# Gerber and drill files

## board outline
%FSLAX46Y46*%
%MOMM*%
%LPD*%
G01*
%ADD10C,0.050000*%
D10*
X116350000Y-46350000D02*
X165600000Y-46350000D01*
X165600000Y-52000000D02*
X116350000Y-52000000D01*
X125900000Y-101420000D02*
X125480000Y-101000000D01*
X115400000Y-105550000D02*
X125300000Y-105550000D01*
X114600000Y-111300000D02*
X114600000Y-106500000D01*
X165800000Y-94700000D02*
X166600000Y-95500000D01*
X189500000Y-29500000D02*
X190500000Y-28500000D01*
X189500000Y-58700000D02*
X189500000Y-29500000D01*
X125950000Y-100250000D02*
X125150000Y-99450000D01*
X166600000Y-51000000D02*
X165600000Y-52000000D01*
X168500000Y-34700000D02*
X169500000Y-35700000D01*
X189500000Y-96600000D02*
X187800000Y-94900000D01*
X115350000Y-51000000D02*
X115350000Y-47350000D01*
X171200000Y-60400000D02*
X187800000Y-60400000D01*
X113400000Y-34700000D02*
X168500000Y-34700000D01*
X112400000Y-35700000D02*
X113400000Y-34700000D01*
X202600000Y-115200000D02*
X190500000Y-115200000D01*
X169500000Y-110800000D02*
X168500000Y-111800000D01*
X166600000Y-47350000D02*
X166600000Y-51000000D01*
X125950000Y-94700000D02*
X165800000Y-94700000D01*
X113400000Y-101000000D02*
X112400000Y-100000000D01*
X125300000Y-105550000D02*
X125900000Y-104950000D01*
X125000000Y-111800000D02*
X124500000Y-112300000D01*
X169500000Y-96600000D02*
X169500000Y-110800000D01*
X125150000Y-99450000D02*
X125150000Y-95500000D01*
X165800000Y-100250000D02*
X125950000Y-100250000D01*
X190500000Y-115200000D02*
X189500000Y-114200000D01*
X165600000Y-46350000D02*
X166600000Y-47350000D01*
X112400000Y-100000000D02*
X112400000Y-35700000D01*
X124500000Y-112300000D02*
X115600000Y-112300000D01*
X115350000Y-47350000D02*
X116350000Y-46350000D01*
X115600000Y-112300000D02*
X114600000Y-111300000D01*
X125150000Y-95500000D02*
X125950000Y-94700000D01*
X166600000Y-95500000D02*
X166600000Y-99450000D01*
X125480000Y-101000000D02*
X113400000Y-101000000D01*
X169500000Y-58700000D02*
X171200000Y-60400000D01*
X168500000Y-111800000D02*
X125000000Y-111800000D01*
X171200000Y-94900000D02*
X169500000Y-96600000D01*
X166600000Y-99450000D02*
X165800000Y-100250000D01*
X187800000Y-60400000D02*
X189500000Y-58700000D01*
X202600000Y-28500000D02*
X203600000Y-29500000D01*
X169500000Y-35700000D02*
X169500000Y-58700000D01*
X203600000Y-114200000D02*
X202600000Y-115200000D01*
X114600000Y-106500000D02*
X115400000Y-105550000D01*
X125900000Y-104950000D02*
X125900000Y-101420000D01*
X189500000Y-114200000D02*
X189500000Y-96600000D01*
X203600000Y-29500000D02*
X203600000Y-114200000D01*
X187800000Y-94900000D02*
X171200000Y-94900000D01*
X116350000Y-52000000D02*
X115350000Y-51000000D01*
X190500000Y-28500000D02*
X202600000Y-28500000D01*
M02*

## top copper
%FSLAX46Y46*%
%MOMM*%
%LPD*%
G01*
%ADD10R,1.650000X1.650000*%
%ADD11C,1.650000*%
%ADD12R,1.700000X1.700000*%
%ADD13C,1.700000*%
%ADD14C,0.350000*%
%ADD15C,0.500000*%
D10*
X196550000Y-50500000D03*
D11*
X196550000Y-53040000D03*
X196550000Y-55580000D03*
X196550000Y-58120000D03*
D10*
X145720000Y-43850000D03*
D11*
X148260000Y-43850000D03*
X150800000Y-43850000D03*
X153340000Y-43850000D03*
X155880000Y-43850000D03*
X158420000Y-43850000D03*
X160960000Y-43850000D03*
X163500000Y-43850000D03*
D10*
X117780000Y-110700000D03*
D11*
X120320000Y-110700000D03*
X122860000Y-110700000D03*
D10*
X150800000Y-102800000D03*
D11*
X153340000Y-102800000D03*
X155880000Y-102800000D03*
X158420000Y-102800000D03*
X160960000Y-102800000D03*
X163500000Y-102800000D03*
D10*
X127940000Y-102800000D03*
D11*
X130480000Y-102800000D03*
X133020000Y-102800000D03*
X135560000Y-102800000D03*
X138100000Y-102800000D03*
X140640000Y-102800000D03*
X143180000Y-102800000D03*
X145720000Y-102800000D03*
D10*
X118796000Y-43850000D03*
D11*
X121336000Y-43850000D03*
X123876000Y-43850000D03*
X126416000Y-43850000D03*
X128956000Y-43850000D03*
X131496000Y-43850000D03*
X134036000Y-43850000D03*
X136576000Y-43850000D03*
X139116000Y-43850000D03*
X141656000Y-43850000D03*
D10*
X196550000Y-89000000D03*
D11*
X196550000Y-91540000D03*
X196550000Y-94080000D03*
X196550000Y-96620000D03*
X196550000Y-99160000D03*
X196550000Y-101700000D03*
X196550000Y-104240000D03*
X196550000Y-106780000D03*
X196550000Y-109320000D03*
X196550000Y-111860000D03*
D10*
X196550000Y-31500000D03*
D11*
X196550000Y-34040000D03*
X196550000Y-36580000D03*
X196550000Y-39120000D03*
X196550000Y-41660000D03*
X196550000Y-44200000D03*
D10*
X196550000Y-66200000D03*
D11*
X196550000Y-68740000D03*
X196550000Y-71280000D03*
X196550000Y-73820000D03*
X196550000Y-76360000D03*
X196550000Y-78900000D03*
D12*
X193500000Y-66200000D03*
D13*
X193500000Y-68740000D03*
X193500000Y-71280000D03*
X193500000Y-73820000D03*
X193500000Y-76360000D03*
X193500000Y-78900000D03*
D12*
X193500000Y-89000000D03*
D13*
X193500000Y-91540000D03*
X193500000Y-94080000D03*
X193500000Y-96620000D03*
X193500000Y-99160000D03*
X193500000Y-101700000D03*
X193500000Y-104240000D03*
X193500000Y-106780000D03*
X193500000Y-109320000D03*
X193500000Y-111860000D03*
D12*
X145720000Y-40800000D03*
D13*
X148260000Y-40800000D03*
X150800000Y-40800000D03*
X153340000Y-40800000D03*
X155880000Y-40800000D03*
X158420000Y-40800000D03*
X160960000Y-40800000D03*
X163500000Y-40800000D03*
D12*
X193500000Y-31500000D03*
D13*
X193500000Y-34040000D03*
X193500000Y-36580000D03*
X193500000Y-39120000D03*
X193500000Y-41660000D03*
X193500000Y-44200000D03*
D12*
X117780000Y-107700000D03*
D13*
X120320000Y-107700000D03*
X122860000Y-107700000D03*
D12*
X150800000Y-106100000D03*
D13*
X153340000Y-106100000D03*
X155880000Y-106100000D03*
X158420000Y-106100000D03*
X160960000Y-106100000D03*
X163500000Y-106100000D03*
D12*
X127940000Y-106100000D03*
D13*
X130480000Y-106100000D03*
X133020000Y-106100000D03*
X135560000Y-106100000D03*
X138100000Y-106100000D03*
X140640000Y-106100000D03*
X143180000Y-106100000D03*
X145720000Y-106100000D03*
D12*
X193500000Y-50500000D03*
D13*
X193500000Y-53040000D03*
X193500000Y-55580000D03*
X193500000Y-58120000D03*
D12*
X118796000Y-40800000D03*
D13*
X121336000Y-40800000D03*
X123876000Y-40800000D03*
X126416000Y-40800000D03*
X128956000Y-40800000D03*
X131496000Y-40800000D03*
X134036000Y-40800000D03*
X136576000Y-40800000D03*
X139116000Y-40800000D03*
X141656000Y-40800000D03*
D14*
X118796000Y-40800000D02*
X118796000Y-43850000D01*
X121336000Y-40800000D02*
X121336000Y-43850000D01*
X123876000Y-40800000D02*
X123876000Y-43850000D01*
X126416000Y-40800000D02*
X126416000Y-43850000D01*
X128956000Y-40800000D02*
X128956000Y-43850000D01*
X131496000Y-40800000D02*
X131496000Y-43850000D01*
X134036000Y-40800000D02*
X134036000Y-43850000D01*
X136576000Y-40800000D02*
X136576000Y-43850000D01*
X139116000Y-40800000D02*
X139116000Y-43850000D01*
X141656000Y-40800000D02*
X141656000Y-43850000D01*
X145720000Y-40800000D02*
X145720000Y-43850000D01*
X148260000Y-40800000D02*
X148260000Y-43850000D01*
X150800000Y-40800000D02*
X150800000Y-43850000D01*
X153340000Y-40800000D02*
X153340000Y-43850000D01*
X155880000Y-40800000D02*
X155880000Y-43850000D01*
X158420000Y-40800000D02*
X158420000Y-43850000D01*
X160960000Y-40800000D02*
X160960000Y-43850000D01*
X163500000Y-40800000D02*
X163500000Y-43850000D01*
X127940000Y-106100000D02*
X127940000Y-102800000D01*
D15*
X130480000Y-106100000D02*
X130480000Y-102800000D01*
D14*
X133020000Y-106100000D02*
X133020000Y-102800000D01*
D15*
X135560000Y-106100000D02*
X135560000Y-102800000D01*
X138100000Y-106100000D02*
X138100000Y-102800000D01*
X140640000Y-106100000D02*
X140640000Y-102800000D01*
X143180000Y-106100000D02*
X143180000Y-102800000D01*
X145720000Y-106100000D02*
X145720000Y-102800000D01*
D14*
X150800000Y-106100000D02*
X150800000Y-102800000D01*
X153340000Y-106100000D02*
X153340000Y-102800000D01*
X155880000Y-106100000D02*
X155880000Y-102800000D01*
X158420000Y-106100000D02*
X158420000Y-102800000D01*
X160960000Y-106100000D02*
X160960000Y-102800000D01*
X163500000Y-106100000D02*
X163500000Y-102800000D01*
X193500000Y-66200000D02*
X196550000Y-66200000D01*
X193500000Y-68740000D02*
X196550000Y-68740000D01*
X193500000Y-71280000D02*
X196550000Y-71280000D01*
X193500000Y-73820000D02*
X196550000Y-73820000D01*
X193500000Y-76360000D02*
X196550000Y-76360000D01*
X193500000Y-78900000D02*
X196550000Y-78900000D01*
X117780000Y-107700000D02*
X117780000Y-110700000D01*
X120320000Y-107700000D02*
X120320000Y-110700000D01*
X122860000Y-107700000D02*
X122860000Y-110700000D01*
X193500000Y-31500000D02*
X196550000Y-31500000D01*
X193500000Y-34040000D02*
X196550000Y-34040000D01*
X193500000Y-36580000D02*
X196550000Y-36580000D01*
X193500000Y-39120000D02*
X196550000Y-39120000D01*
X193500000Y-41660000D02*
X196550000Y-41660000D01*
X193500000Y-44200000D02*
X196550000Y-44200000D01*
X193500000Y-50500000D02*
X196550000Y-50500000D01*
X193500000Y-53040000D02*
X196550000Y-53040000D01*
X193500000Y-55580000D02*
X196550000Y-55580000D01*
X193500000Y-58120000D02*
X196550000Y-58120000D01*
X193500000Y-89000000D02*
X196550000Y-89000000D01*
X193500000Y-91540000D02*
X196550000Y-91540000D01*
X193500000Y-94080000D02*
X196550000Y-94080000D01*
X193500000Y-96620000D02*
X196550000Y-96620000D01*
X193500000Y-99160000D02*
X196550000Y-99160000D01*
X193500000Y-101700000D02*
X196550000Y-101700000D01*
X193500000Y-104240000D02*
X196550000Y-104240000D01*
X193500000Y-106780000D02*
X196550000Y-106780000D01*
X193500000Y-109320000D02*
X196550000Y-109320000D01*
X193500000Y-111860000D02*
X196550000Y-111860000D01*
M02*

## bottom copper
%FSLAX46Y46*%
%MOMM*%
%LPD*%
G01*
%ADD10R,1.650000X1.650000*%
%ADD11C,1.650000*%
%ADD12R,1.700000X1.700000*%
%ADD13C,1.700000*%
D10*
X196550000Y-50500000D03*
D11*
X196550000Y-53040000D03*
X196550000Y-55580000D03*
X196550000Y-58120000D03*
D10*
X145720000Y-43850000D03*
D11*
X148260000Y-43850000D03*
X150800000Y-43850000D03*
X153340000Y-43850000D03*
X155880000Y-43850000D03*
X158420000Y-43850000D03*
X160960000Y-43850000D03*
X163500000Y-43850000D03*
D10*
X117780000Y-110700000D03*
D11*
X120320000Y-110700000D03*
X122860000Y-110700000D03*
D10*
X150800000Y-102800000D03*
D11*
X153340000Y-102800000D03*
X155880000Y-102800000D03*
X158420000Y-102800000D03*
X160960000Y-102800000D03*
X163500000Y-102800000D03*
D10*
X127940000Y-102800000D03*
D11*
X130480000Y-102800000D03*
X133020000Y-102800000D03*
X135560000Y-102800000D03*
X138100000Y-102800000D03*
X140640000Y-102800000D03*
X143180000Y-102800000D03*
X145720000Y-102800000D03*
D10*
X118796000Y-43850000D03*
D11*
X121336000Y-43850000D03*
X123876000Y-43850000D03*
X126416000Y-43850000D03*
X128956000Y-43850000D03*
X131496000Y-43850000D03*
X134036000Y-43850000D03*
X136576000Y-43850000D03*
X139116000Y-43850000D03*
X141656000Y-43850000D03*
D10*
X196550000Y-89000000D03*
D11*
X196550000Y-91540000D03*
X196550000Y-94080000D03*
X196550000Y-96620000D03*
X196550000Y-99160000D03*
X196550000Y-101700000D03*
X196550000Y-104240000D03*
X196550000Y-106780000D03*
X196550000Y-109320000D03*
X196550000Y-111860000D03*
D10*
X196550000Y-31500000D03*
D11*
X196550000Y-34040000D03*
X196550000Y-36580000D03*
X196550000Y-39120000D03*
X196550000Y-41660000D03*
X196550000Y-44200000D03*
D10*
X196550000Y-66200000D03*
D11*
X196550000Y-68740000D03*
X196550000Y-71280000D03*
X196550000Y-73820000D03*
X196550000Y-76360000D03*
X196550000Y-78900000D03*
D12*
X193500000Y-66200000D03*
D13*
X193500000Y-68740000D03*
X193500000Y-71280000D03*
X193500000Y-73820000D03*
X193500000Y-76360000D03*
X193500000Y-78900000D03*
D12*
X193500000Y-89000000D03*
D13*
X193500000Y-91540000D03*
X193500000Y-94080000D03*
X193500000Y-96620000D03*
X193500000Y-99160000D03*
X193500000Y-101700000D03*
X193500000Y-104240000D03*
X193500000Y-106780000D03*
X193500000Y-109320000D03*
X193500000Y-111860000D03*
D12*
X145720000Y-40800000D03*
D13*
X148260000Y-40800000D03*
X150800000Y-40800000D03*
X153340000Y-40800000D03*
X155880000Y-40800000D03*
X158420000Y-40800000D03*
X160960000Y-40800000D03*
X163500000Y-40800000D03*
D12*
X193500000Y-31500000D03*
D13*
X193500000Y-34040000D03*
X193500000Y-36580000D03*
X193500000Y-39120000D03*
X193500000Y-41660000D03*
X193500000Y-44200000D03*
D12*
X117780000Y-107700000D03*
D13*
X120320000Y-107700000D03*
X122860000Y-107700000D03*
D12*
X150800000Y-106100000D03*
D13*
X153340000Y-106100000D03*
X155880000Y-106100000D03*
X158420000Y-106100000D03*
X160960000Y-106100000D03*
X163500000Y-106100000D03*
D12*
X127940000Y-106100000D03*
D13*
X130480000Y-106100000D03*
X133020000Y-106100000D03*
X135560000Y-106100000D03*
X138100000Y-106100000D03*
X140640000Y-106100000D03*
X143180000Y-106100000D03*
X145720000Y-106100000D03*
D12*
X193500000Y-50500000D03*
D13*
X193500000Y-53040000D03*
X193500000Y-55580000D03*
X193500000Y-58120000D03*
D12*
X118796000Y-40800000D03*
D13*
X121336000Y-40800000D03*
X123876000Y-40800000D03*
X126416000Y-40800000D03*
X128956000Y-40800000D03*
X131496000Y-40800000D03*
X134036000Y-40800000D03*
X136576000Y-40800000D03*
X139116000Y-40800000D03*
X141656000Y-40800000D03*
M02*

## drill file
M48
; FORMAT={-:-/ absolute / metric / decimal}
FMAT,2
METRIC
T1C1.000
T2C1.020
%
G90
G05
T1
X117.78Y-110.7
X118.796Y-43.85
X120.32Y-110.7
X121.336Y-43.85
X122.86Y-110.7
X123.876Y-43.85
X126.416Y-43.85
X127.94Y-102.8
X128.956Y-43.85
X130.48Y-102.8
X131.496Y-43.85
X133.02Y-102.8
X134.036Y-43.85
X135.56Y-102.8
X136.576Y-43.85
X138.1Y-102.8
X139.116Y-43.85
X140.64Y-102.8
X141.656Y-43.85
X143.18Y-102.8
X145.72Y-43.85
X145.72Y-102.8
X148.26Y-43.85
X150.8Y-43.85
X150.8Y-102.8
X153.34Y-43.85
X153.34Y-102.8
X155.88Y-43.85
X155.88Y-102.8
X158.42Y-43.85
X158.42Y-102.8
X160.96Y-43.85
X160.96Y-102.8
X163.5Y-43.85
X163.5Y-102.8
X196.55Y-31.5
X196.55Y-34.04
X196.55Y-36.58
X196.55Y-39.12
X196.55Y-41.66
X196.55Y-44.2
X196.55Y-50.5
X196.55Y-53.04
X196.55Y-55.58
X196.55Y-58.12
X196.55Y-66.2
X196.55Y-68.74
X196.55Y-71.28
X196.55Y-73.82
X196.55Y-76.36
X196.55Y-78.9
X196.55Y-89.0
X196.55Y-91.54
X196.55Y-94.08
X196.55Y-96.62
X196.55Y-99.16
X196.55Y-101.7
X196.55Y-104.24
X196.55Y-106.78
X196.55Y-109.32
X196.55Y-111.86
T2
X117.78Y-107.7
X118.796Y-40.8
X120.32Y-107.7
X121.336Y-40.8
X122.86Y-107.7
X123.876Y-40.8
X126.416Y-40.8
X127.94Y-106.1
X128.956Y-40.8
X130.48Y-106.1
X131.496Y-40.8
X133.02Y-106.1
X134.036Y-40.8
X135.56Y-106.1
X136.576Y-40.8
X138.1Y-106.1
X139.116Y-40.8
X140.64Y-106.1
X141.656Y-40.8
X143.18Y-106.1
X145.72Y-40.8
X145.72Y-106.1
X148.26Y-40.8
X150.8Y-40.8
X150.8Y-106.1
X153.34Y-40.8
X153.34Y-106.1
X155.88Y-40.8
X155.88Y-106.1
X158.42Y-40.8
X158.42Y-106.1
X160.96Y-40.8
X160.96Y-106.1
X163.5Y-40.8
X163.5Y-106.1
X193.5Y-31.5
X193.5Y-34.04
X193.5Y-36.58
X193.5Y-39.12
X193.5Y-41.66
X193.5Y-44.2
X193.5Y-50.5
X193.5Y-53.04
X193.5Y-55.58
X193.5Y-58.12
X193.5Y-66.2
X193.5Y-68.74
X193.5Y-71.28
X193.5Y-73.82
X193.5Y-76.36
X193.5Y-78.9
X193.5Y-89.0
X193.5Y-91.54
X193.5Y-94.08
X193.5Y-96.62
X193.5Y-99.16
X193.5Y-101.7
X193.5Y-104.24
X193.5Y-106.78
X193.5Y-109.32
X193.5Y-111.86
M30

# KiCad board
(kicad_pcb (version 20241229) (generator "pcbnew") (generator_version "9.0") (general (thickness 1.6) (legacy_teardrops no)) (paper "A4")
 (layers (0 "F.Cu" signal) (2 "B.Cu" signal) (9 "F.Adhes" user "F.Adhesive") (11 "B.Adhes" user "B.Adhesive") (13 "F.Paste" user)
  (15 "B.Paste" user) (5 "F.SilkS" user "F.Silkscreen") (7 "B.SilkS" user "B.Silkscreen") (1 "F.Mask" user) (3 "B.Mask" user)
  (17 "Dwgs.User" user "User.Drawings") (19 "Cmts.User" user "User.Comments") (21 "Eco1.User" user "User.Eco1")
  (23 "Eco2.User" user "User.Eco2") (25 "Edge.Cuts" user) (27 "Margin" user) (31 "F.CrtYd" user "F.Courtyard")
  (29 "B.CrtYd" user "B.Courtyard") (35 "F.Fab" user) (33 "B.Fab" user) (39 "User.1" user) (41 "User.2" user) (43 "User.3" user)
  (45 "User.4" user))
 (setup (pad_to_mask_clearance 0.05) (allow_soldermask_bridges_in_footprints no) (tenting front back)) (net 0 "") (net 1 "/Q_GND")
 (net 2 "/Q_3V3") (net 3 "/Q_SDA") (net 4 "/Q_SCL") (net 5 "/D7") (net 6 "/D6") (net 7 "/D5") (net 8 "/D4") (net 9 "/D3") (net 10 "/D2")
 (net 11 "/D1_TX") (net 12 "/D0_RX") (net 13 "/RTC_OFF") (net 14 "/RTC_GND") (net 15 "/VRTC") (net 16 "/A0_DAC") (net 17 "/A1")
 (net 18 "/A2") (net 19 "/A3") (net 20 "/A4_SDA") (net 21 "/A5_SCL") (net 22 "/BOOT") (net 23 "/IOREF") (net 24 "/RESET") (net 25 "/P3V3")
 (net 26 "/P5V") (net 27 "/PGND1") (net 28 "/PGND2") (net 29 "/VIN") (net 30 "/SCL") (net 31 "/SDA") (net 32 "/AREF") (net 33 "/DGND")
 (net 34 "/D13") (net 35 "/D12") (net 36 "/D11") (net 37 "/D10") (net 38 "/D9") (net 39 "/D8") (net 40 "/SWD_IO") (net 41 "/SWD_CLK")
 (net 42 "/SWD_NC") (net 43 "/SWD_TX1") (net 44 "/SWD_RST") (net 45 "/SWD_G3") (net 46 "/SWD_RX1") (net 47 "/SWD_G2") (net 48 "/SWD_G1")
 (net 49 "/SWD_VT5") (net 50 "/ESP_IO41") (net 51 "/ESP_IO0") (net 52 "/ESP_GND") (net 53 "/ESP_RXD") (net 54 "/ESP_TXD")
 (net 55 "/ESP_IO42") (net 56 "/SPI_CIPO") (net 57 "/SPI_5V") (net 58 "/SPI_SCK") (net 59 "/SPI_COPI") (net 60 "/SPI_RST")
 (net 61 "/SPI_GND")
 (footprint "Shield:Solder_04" (layer "F.Cu") (at 196.55 50.5)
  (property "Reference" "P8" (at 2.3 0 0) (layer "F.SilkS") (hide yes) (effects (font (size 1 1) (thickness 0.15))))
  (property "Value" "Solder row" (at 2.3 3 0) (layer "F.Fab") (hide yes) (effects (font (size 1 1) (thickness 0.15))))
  (pad "1" thru_hole rect (at 0 0) (size 1.65 1.65) (drill 1) (layers "*.Cu" "*.Mask") (remove_unused_layers no) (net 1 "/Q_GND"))
  (pad "2" thru_hole circle (at 0 2.54) (size 1.65 1.65) (drill 1) (layers "*.Cu" "*.Mask") (remove_unused_layers no) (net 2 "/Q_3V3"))
  (pad "3" thru_hole circle (at 0 5.08) (size 1.65 1.65) (drill 1) (layers "*.Cu" "*.Mask") (remove_unused_layers no) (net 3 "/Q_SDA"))
  (pad "4" thru_hole circle (at 0 7.62) (size 1.65 1.65) (drill 1) (layers "*.Cu" "*.Mask") (remove_unused_layers no) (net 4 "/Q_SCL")))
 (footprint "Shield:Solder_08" (layer "F.Cu") (at 145.72 43.85 90)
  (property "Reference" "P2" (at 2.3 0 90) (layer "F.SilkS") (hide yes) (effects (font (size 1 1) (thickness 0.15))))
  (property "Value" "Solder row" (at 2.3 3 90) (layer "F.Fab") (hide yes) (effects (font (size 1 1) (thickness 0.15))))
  (pad "1" thru_hole rect (at 0 0 90) (size 1.65 1.65) (drill 1) (layers "*.Cu" "*.Mask") (remove_unused_layers no) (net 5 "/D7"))
  (pad "2" thru_hole circle (at 0 2.54 90) (size 1.65 1.65) (drill 1) (layers "*.Cu" "*.Mask") (remove_unused_layers no) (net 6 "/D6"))
  (pad "3" thru_hole circle (at 0 5.08 90) (size 1.65 1.65) (drill 1) (layers "*.Cu" "*.Mask") (remove_unused_layers no) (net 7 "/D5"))
  (pad "4" thru_hole circle (at 0 7.62 90) (size 1.65 1.65) (drill 1) (layers "*.Cu" "*.Mask") (remove_unused_layers no) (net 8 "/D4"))
  (pad "5" thru_hole circle (at 0 10.16 90) (size 1.65 1.65) (drill 1) (layers "*.Cu" "*.Mask") (remove_unused_layers no) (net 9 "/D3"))
  (pad "6" thru_hole circle (at 0 12.7 90) (size 1.65 1.65) (drill 1) (layers "*.Cu" "*.Mask") (remove_unused_layers no) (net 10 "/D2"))
  (pad "7" thru_hole circle (at 0 15.24 90) (size 1.65 1.65) (drill 1) (layers "*.Cu" "*.Mask") (remove_unused_layers no) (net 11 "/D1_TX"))
  (pad "8" thru_hole circle (at 0 17.78 90) (size 1.65 1.65) (drill 1) (layers "*.Cu" "*.Mask") (remove_unused_layers no) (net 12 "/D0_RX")))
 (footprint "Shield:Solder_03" (layer "F.Cu") (at 117.78 110.7 90)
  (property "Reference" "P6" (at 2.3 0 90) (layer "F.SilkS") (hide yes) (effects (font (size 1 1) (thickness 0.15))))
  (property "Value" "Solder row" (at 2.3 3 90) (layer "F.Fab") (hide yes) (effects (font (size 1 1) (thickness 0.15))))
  (pad "1" thru_hole rect (at 0 0 90) (size 1.65 1.65) (drill 1) (layers "*.Cu" "*.Mask") (remove_unused_layers no) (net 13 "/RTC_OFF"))
  (pad "2" thru_hole circle (at 0 2.54 90) (size 1.65 1.65) (drill 1) (layers "*.Cu" "*.Mask") (remove_unused_layers no) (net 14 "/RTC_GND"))
  (pad "3" thru_hole circle (at 0 5.08 90) (size 1.65 1.65) (drill 1) (layers "*.Cu" "*.Mask") (remove_unused_layers no) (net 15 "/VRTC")))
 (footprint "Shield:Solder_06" (layer "F.Cu") (at 150.8 102.8 90)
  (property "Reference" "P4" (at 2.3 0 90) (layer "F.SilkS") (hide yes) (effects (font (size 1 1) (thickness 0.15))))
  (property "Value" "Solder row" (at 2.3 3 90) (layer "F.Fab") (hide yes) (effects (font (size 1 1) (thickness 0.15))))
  (pad "1" thru_hole rect (at 0 0 90) (size 1.65 1.65) (drill 1) (layers "*.Cu" "*.Mask") (remove_unused_layers no) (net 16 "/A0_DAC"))
  (pad "2" thru_hole circle (at 0 2.54 90) (size 1.65 1.65) (drill 1) (layers "*.Cu" "*.Mask") (remove_unused_layers no) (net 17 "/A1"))
  (pad "3" thru_hole circle (at 0 5.08 90) (size 1.65 1.65) (drill 1) (layers "*.Cu" "*.Mask") (remove_unused_layers no) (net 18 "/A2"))
  (pad "4" thru_hole circle (at 0 7.62 90) (size 1.65 1.65) (drill 1) (layers "*.Cu" "*.Mask") (remove_unused_layers no) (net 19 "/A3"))
  (pad "5" thru_hole circle (at 0 10.16 90) (size 1.65 1.65) (drill 1) (layers "*.Cu" "*.Mask") (remove_unused_layers no) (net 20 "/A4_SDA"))
  (pad "6" thru_hole circle (at 0 12.7 90) (size 1.65 1.65) (drill 1) (layers "*.Cu" "*.Mask") (remove_unused_layers no) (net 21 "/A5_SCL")))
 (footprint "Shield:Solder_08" (layer "F.Cu") (at 127.94 102.8 90)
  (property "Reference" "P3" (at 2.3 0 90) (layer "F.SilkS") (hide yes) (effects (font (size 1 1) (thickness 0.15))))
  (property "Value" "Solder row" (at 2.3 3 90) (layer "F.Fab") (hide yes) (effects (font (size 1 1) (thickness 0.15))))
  (pad "1" thru_hole rect (at 0 0 90) (size 1.65 1.65) (drill 1) (layers "*.Cu" "*.Mask") (remove_unused_layers no) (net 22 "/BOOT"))
  (pad "2" thru_hole circle (at 0 2.54 90) (size 1.65 1.65) (drill 1) (layers "*.Cu" "*.Mask") (remove_unused_layers no) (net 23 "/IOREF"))
  (pad "3" thru_hole circle (at 0 5.08 90) (size 1.65 1.65) (drill 1) (layers "*.Cu" "*.Mask") (remove_unused_layers no) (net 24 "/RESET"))
  (pad "4" thru_hole circle (at 0 7.62 90) (size 1.65 1.65) (drill 1) (layers "*.Cu" "*.Mask") (remove_unused_layers no) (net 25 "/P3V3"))
  (pad "5" thru_hole circle (at 0 10.16 90) (size 1.65 1.65) (drill 1) (layers "*.Cu" "*.Mask") (remove_unused_layers no) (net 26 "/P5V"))
  (pad "6" thru_hole circle (at 0 12.7 90) (size 1.65 1.65) (drill 1) (layers "*.Cu" "*.Mask") (remove_unused_layers no) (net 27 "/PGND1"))
  (pad "7" thru_hole circle (at 0 15.24 90) (size 1.65 1.65) (drill 1) (layers "*.Cu" "*.Mask") (remove_unused_layers no) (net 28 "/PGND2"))
  (pad "8" thru_hole circle (at 0 17.78 90) (size 1.65 1.65) (drill 1) (layers "*.Cu" "*.Mask") (remove_unused_layers no) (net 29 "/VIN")))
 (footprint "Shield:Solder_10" (layer "F.Cu") (at 118.796 43.85 90)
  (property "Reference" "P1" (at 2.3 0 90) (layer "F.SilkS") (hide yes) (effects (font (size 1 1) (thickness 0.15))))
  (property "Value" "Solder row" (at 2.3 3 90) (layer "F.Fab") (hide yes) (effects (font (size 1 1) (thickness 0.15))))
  (pad "1" thru_hole rect (at 0 0 90) (size 1.65 1.65) (drill 1) (layers "*.Cu" "*.Mask") (remove_unused_layers no) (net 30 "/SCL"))
  (pad "2" thru_hole circle (at 0 2.54 90) (size 1.65 1.65) (drill 1) (layers "*.Cu" "*.Mask") (remove_unused_layers no) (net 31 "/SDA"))
  (pad "3" thru_hole circle (at 0 5.08 90) (size 1.65 1.65) (drill 1) (layers "*.Cu" "*.Mask") (remove_unused_layers no) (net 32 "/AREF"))
  (pad "4" thru_hole circle (at 0 7.62 90) (size 1.65 1.65) (drill 1) (layers "*.Cu" "*.Mask") (remove_unused_layers no) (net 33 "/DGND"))
  (pad "5" thru_hole circle (at 0 10.16 90) (size 1.65 1.65) (drill 1) (layers "*.Cu" "*.Mask") (remove_unused_layers no) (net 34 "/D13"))
  (pad "6" thru_hole circle (at 0 12.7 90) (size 1.65 1.65) (drill 1) (layers "*.Cu" "*.Mask") (remove_unused_layers no) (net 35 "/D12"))
  (pad "7" thru_hole circle (at 0 15.24 90) (size 1.65 1.65) (drill 1) (layers "*.Cu" "*.Mask") (remove_unused_layers no) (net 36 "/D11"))
  (pad "8" thru_hole circle (at 0 17.78 90) (size 1.65 1.65) (drill 1) (layers "*.Cu" "*.Mask") (remove_unused_layers no) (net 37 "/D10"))
  (pad "9" thru_hole circle (at 0 20.32 90) (size 1.65 1.65) (drill 1) (layers "*.Cu" "*.Mask") (remove_unused_layers no) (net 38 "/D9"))
  (pad "10" thru_hole circle (at 0 22.86 90) (size 1.65 1.65) (drill 1) (layers "*.Cu" "*.Mask") (remove_unused_layers no) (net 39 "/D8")))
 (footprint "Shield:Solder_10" (layer "F.Cu") (at 196.55 89)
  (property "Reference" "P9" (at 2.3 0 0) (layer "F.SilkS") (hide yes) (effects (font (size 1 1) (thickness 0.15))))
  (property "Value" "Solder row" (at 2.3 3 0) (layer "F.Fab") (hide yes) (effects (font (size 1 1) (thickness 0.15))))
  (pad "1" thru_hole rect (at 0 0) (size 1.65 1.65) (drill 1) (layers "*.Cu" "*.Mask") (remove_unused_layers no) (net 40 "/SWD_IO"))
  (pad "2" thru_hole circle (at 0 2.54) (size 1.65 1.65) (drill 1) (layers "*.Cu" "*.Mask") (remove_unused_layers no) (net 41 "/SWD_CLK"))
  (pad "3" thru_hole circle (at 0 5.08) (size 1.65 1.65) (drill 1) (layers "*.Cu" "*.Mask") (remove_unused_layers no) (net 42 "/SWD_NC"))
  (pad "4" thru_hole circle (at 0 7.62) (size 1.65 1.65) (drill 1) (layers "*.Cu" "*.Mask") (remove_unused_layers no) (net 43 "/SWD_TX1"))
  (pad "5" thru_hole circle (at 0 10.16) (size 1.65 1.65) (drill 1) (layers "*.Cu" "*.Mask") (remove_unused_layers no) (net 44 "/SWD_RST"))
  (pad "6" thru_hole circle (at 0 12.7) (size 1.65 1.65) (drill 1) (layers "*.Cu" "*.Mask") (remove_unused_layers no) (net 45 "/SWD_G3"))
  (pad "7" thru_hole circle (at 0 15.24) (size 1.65 1.65) (drill 1) (layers "*.Cu" "*.Mask") (remove_unused_layers no) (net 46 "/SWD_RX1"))
  (pad "8" thru_hole circle (at 0 17.78) (size 1.65 1.65) (drill 1) (layers "*.Cu" "*.Mask") (remove_unused_layers no) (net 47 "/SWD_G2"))
  (pad "9" thru_hole circle (at 0 20.32) (size 1.65 1.65) (drill 1) (layers "*.Cu" "*.Mask") (remove_unused_layers no) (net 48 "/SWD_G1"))
  (pad "10" thru_hole circle (at 0 22.86) (size 1.65 1.65) (drill 1) (layers "*.Cu" "*.Mask") (remove_unused_layers no) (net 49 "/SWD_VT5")))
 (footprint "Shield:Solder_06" (layer "F.Cu") (at 196.55 31.5)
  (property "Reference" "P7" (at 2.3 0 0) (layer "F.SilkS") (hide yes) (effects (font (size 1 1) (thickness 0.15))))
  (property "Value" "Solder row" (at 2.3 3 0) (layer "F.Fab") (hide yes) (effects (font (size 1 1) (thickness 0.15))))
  (pad "1" thru_hole rect (at 0 0) (size 1.65 1.65) (drill 1) (layers "*.Cu" "*.Mask") (remove_unused_layers no) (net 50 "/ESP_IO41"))
  (pad "2" thru_hole circle (at 0 2.54) (size 1.65 1.65) (drill 1) (layers "*.Cu" "*.Mask") (remove_unused_layers no) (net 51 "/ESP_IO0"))
  (pad "3" thru_hole circle (at 0 5.08) (size 1.65 1.65) (drill 1) (layers "*.Cu" "*.Mask") (remove_unused_layers no) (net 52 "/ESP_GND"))
  (pad "4" thru_hole circle (at 0 7.62) (size 1.65 1.65) (drill 1) (layers "*.Cu" "*.Mask") (remove_unused_layers no) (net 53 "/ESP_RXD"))
  (pad "5" thru_hole circle (at 0 10.16) (size 1.65 1.65) (drill 1) (layers "*.Cu" "*.Mask") (remove_unused_layers no) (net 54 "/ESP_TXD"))
  (pad "6" thru_hole circle (at 0 12.7) (size 1.65 1.65) (drill 1) (layers "*.Cu" "*.Mask") (remove_unused_layers no) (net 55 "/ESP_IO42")))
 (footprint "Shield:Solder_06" (layer "F.Cu") (at 196.55 66.2)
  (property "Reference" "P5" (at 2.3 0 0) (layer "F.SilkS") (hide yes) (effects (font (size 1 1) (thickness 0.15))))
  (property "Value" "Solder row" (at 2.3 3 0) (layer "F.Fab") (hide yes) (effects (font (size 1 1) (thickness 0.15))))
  (pad "1" thru_hole rect (at 0 0) (size 1.65 1.65) (drill 1) (layers "*.Cu" "*.Mask") (remove_unused_layers no) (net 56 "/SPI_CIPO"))
  (pad "2" thru_hole circle (at 0 2.54) (size 1.65 1.65) (drill 1) (layers "*.Cu" "*.Mask") (remove_unused_layers no) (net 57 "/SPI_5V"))
  (pad "3" thru_hole circle (at 0 5.08) (size 1.65 1.65) (drill 1) (layers "*.Cu" "*.Mask") (remove_unused_layers no) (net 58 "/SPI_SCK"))
  (pad "4" thru_hole circle (at 0 7.62) (size 1.65 1.65) (drill 1) (layers "*.Cu" "*.Mask") (remove_unused_layers no) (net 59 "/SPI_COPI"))
  (pad "5" thru_hole circle (at 0 10.16) (size 1.65 1.65) (drill 1) (layers "*.Cu" "*.Mask") (remove_unused_layers no) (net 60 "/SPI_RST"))
  (pad "6" thru_hole circle (at 0 12.7) (size 1.65 1.65) (drill 1) (layers "*.Cu" "*.Mask") (remove_unused_layers no) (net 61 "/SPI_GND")))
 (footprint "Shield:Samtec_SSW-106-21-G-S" (layer "B.Cu") (at 193.5 66.2 180)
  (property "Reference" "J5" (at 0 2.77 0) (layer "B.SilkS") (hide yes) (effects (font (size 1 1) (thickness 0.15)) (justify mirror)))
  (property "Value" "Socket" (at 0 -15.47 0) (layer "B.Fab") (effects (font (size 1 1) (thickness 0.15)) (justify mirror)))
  (pad "1" thru_hole rect (at 0 0 180) (size 1.7 1.7) (drill 1.02) (layers "*.Cu" "*.Mask") (remove_unused_layers no) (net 56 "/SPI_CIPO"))
  (pad "2" thru_hole circle (at 0 -2.54 180) (size 1.7 1.7) (drill 1.02) (layers "*.Cu" "*.Mask") (remove_unused_layers no)
   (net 57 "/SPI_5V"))
  (pad "3" thru_hole circle (at 0 -5.08 180) (size 1.7 1.7) (drill 1.02) (layers "*.Cu" "*.Mask") (remove_unused_layers no)
   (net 58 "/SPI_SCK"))
  (pad "4" thru_hole circle (at 0 -7.62 180) (size 1.7 1.7) (drill 1.02) (layers "*.Cu" "*.Mask") (remove_unused_layers no)
   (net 59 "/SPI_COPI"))
  (pad "5" thru_hole circle (at 0 -10.16 180) (size 1.7 1.7) (drill 1.02) (layers "*.Cu" "*.Mask") (remove_unused_layers no)
   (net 60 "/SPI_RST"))
  (pad "6" thru_hole circle (at 0 -12.7 180) (size 1.7 1.7) (drill 1.02) (layers "*.Cu" "*.Mask") (remove_unused_layers no)
   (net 61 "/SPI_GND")))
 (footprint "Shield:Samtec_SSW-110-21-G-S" (layer "B.Cu") (at 193.5 89 180)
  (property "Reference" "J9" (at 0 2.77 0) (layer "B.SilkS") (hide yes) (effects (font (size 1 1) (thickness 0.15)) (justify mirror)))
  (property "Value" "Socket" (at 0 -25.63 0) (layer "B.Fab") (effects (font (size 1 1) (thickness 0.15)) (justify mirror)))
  (pad "1" thru_hole rect (at 0 0 180) (size 1.7 1.7) (drill 1.02) (layers "*.Cu" "*.Mask") (remove_unused_layers no) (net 40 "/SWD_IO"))
  (pad "2" thru_hole circle (at 0 -2.54 180) (size 1.7 1.7) (drill 1.02) (layers "*.Cu" "*.Mask") (remove_unused_layers no)
   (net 41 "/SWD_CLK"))
  (pad "3" thru_hole circle (at 0 -5.08 180) (size 1.7 1.7) (drill 1.02) (layers "*.Cu" "*.Mask") (remove_unused_layers no)
   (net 42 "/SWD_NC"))
  (pad "4" thru_hole circle (at 0 -7.62 180) (size 1.7 1.7) (drill 1.02) (layers "*.Cu" "*.Mask") (remove_unused_layers no)
   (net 43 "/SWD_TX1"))
  (pad "5" thru_hole circle (at 0 -10.16 180) (size 1.7 1.7) (drill 1.02) (layers "*.Cu" "*.Mask") (remove_unused_layers no)
   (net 44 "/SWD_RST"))
  (pad "6" thru_hole circle (at 0 -12.7 180) (size 1.7 1.7) (drill 1.02) (layers "*.Cu" "*.Mask") (remove_unused_layers no)
   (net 45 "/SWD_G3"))
  (pad "7" thru_hole circle (at 0 -15.24 180) (size 1.7 1.7) (drill 1.02) (layers "*.Cu" "*.Mask") (remove_unused_layers no)
   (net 46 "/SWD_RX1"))
  (pad "8" thru_hole circle (at 0 -17.78 180) (size 1.7 1.7) (drill 1.02) (layers "*.Cu" "*.Mask") (remove_unused_layers no)
   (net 47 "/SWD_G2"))
  (pad "9" thru_hole circle (at 0 -20.32 180) (size 1.7 1.7) (drill 1.02) (layers "*.Cu" "*.Mask") (remove_unused_layers no)
   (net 48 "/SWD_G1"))
  (pad "10" thru_hole circle (at 0 -22.86 180) (size 1.7 1.7) (drill 1.02) (layers "*.Cu" "*.Mask") (remove_unused_layers no)
   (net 49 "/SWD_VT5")))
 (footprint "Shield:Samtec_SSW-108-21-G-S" (layer "B.Cu") (at 145.72 40.8 -90)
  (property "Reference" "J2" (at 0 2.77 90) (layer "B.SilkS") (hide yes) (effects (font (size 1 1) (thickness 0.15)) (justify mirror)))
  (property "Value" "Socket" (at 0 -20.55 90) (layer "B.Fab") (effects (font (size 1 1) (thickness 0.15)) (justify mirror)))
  (pad "1" thru_hole rect (at 0 0 270) (size 1.7 1.7) (drill 1.02) (layers "*.Cu" "*.Mask") (remove_unused_layers no) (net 5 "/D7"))
  (pad "2" thru_hole circle (at 0 -2.54 270) (size 1.7 1.7) (drill 1.02) (layers "*.Cu" "*.Mask") (remove_unused_layers no) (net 6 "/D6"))
  (pad "3" thru_hole circle (at 0 -5.08 270) (size 1.7 1.7) (drill 1.02) (layers "*.Cu" "*.Mask") (remove_unused_layers no) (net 7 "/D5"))
  (pad "4" thru_hole circle (at 0 -7.62 270) (size 1.7 1.7) (drill 1.02) (layers "*.Cu" "*.Mask") (remove_unused_layers no) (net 8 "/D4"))
  (pad "5" thru_hole circle (at 0 -10.16 270) (size 1.7 1.7) (drill 1.02) (layers "*.Cu" "*.Mask") (remove_unused_layers no) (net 9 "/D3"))
  (pad "6" thru_hole circle (at 0 -12.7 270) (size 1.7 1.7) (drill 1.02) (layers "*.Cu" "*.Mask") (remove_unused_layers no) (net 10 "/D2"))
  (pad "7" thru_hole circle (at 0 -15.24 270) (size 1.7 1.7) (drill 1.02) (layers "*.Cu" "*.Mask") (remove_unused_layers no)
   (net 11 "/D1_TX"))
  (pad "8" thru_hole circle (at 0 -17.78 270) (size 1.7 1.7) (drill 1.02) (layers "*.Cu" "*.Mask") (remove_unused_layers no)
   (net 12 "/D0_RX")))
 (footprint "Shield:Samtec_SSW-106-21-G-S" (layer "B.Cu") (at 193.5 31.5 180)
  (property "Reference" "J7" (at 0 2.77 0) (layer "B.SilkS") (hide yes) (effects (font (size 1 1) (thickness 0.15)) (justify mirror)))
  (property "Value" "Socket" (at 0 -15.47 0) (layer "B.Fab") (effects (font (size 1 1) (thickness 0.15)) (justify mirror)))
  (pad "1" thru_hole rect (at 0 0 180) (size 1.7 1.7) (drill 1.02) (layers "*.Cu" "*.Mask") (remove_unused_layers no) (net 50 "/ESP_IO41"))
  (pad "2" thru_hole circle (at 0 -2.54 180) (size 1.7 1.7) (drill 1.02) (layers "*.Cu" "*.Mask") (remove_unused_layers no)
   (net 51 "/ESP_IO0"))
  (pad "3" thru_hole circle (at 0 -5.08 180) (size 1.7 1.7) (drill 1.02) (layers "*.Cu" "*.Mask") (remove_unused_layers no)
   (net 52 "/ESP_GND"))
  (pad "4" thru_hole circle (at 0 -7.62 180) (size 1.7 1.7) (drill 1.02) (layers "*.Cu" "*.Mask") (remove_unused_layers no)
   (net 53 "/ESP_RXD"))
  (pad "5" thru_hole circle (at 0 -10.16 180) (size 1.7 1.7) (drill 1.02) (layers "*.Cu" "*.Mask") (remove_unused_layers no)
   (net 54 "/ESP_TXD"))
  (pad "6" thru_hole circle (at 0 -12.7 180) (size 1.7 1.7) (drill 1.02) (layers "*.Cu" "*.Mask") (remove_unused_layers no)
   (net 55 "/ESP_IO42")))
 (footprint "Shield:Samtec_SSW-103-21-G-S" (layer "B.Cu") (at 117.78 107.7 -90)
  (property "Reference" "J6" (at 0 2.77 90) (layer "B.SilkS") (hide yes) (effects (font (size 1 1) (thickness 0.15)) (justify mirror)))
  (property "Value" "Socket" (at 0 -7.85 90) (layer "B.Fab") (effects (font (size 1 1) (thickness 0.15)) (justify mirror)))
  (pad "1" thru_hole rect (at 0 0 270) (size 1.7 1.7) (drill 1.02) (layers "*.Cu" "*.Mask") (remove_unused_layers no) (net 13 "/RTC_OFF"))
  (pad "2" thru_hole circle (at 0 -2.54 270) (size 1.7 1.7) (drill 1.02) (layers "*.Cu" "*.Mask") (remove_unused_layers no)
   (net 14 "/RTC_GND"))
  (pad "3" thru_hole circle (at 0 -5.08 270) (size 1.7 1.7) (drill 1.02) (layers "*.Cu" "*.Mask") (remove_unused_layers no) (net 15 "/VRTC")))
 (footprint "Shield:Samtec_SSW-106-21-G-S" (layer "B.Cu") (at 150.8 106.1 -90)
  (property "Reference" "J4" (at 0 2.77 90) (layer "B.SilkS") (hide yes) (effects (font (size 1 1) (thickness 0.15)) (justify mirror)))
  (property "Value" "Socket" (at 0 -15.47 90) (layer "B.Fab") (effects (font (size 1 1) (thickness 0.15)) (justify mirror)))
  (pad "1" thru_hole rect (at 0 0 270) (size 1.7 1.7) (drill 1.02) (layers "*.Cu" "*.Mask") (remove_unused_layers no) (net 16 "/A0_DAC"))
  (pad "2" thru_hole circle (at 0 -2.54 270) (size 1.7 1.7) (drill 1.02) (layers "*.Cu" "*.Mask") (remove_unused_layers no) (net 17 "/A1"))
  (pad "3" thru_hole circle (at 0 -5.08 270) (size 1.7 1.7) (drill 1.02) (layers "*.Cu" "*.Mask") (remove_unused_layers no) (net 18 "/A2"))
  (pad "4" thru_hole circle (at 0 -7.62 270) (size 1.7 1.7) (drill 1.02) (layers "*.Cu" "*.Mask") (remove_unused_layers no) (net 19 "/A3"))
  (pad "5" thru_hole circle (at 0 -10.16 270) (size 1.7 1.7) (drill 1.02) (layers "*.Cu" "*.Mask") (remove_unused_layers no)
   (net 20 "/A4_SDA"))
  (pad "6" thru_hole circle (at 0 -12.7 270) (size 1.7 1.7) (drill 1.02) (layers "*.Cu" "*.Mask") (remove_unused_layers no)
   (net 21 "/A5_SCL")))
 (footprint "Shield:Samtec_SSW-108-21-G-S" (layer "B.Cu") (at 127.94 106.1 -90)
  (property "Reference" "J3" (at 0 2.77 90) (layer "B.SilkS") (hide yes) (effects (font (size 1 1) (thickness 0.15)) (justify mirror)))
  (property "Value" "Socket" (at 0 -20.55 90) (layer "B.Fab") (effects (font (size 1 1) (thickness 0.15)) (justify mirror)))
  (pad "1" thru_hole rect (at 0 0 270) (size 1.7 1.7) (drill 1.02) (layers "*.Cu" "*.Mask") (remove_unused_layers no) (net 22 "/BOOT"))
  (pad "2" thru_hole circle (at 0 -2.54 270) (size 1.7 1.7) (drill 1.02) (layers "*.Cu" "*.Mask") (remove_unused_layers no)
   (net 23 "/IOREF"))
  (pad "3" thru_hole circle (at 0 -5.08 270) (size 1.7 1.7) (drill 1.02) (layers "*.Cu" "*.Mask") (remove_unused_layers no)
   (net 24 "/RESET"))
  (pad "4" thru_hole circle (at 0 -7.62 270) (size 1.7 1.7) (drill 1.02) (layers "*.Cu" "*.Mask") (remove_unused_layers no) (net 25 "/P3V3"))
  (pad "5" thru_hole circle (at 0 -10.16 270) (size 1.7 1.7) (drill 1.02) (layers "*.Cu" "*.Mask") (remove_unused_layers no) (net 26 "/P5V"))
  (pad "6" thru_hole circle (at 0 -12.7 270) (size 1.7 1.7) (drill 1.02) (layers "*.Cu" "*.Mask") (remove_unused_layers no)
   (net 27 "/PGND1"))
  (pad "7" thru_hole circle (at 0 -15.24 270) (size 1.7 1.7) (drill 1.02) (layers "*.Cu" "*.Mask") (remove_unused_layers no)
   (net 28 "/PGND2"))
  (pad "8" thru_hole circle (at 0 -17.78 270) (size 1.7 1.7) (drill 1.02) (layers "*.Cu" "*.Mask") (remove_unused_layers no) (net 29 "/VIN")))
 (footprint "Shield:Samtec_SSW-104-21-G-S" (layer "B.Cu") (at 193.5 50.5 180)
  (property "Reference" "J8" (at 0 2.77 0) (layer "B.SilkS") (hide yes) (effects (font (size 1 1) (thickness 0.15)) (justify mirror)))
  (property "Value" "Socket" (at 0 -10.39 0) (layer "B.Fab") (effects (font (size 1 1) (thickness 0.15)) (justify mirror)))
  (pad "1" thru_hole rect (at 0 0 180) (size 1.7 1.7) (drill 1.02) (layers "*.Cu" "*.Mask") (remove_unused_layers no) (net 1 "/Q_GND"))
  (pad "2" thru_hole circle (at 0 -2.54 180) (size 1.7 1.7) (drill 1.02) (layers "*.Cu" "*.Mask") (remove_unused_layers no) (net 2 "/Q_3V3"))
  (pad "3" thru_hole circle (at 0 -5.08 180) (size 1.7 1.7) (drill 1.02) (layers "*.Cu" "*.Mask") (remove_unused_layers no) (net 3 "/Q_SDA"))
  (pad "4" thru_hole circle (at 0 -7.62 180) (size 1.7 1.7) (drill 1.02) (layers "*.Cu" "*.Mask") (remove_unused_layers no) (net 4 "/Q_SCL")))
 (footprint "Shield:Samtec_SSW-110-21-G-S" (layer "B.Cu") (at 118.796 40.8 -90)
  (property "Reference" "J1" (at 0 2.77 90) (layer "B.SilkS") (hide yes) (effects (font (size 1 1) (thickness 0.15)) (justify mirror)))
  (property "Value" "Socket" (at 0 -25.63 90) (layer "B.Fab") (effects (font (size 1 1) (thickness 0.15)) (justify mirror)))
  (pad "1" thru_hole rect (at 0 0 270) (size 1.7 1.7) (drill 1.02) (layers "*.Cu" "*.Mask") (remove_unused_layers no) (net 30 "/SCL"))
  (pad "2" thru_hole circle (at 0 -2.54 270) (size 1.7 1.7) (drill 1.02) (layers "*.Cu" "*.Mask") (remove_unused_layers no) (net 31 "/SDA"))
  (pad "3" thru_hole circle (at 0 -5.08 270) (size 1.7 1.7) (drill 1.02) (layers "*.Cu" "*.Mask") (remove_unused_layers no) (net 32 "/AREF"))
  (pad "4" thru_hole circle (at 0 -7.62 270) (size 1.7 1.7) (drill 1.02) (layers "*.Cu" "*.Mask") (remove_unused_layers no) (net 33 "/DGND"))
  (pad "5" thru_hole circle (at 0 -10.16 270) (size 1.7 1.7) (drill 1.02) (layers "*.Cu" "*.Mask") (remove_unused_layers no) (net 34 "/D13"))
  (pad "6" thru_hole circle (at 0 -12.7 270) (size 1.7 1.7) (drill 1.02) (layers "*.Cu" "*.Mask") (remove_unused_layers no) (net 35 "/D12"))
  (pad "7" thru_hole circle (at 0 -15.24 270) (size 1.7 1.7) (drill 1.02) (layers "*.Cu" "*.Mask") (remove_unused_layers no) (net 36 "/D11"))
  (pad "8" thru_hole circle (at 0 -17.78 270) (size 1.7 1.7) (drill 1.02) (layers "*.Cu" "*.Mask") (remove_unused_layers no) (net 37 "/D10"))
  (pad "9" thru_hole circle (at 0 -20.32 270) (size 1.7 1.7) (drill 1.02) (layers "*.Cu" "*.Mask") (remove_unused_layers no) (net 38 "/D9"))
  (pad "10" thru_hole circle (at 0 -22.86 270) (size 1.7 1.7) (drill 1.02) (layers "*.Cu" "*.Mask") (remove_unused_layers no) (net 39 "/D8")))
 (gr_line (start 116.35 46.35) (end 165.6 46.35) (stroke (width 0.05) (type default)) (layer "Edge.Cuts"))
 (gr_line (start 165.6 52) (end 116.35 52) (stroke (width 0.05) (type default)) (layer "Edge.Cuts"))
 (gr_line (start 125.9 101.42) (end 125.48 101) (stroke (width 0.05) (type default)) (layer "Edge.Cuts"))
 (gr_line (start 115.4 105.55) (end 125.3 105.55) (stroke (width 0.05) (type default)) (layer "Edge.Cuts"))
 (gr_line (start 114.6 111.3) (end 114.6 106.5) (stroke (width 0.05) (type default)) (layer "Edge.Cuts"))
 (gr_line (start 165.8 94.7) (end 166.6 95.5) (stroke (width 0.05) (type default)) (layer "Edge.Cuts"))
 (gr_line (start 189.5 29.5) (end 190.5 28.5) (stroke (width 0.05) (type default)) (layer "Edge.Cuts"))
 (gr_line (start 189.5 58.7) (end 189.5 29.5) (stroke (width 0.05) (type default)) (layer "Edge.Cuts"))
 (gr_line (start 125.95 100.25) (end 125.15 99.45) (stroke (width 0.05) (type default)) (layer "Edge.Cuts"))
 (gr_line (start 166.6 51) (end 165.6 52) (stroke (width 0.05) (type default)) (layer "Edge.Cuts"))
 (gr_line (start 168.5 34.7) (end 169.5 35.7) (stroke (width 0.05) (type default)) (layer "Edge.Cuts"))
 (gr_line (start 189.5 96.6) (end 187.8 94.9) (stroke (width 0.05) (type default)) (layer "Edge.Cuts"))
 (gr_line (start 115.35 51) (end 115.35 47.35) (stroke (width 0.05) (type default)) (layer "Edge.Cuts"))
 (gr_line (start 171.2 60.4) (end 187.8 60.4) (stroke (width 0.05) (type default)) (layer "Edge.Cuts"))
 (gr_line (start 113.4 34.7) (end 168.5 34.7) (stroke (width 0.05) (type default)) (layer "Edge.Cuts"))
 (gr_line (start 112.4 35.7) (end 113.4 34.7) (stroke (width 0.05) (type default)) (layer "Edge.Cuts"))
 (gr_line (start 202.6 115.2) (end 190.5 115.2) (stroke (width 0.05) (type default)) (layer "Edge.Cuts"))
 (gr_line (start 169.5 110.8) (end 168.5 111.8) (stroke (width 0.05) (type default)) (layer "Edge.Cuts"))
 (gr_line (start 166.6 47.35) (end 166.6 51) (stroke (width 0.05) (type default)) (layer "Edge.Cuts"))
 (gr_line (start 125.95 94.7) (end 165.8 94.7) (stroke (width 0.05) (type default)) (layer "Edge.Cuts"))
 (gr_line (start 113.4 101) (end 112.4 100) (stroke (width 0.05) (type default)) (layer "Edge.Cuts"))
 (gr_line (start 125.3 105.55) (end 125.9 104.95) (stroke (width 0.05) (type default)) (layer "Edge.Cuts"))
 (gr_line (start 125 111.8) (end 124.5 112.3) (stroke (width 0.05) (type default)) (layer "Edge.Cuts"))
 (gr_line (start 169.5 96.6) (end 169.5 110.8) (stroke (width 0.05) (type default)) (layer "Edge.Cuts"))
 (gr_line (start 125.15 99.45) (end 125.15 95.5) (stroke (width 0.05) (type default)) (layer "Edge.Cuts"))
 (gr_line (start 165.8 100.25) (end 125.95 100.25) (stroke (width 0.05) (type default)) (layer "Edge.Cuts"))
 (gr_line (start 190.5 115.2) (end 189.5 114.2) (stroke (width 0.05) (type default)) (layer "Edge.Cuts"))
 (gr_line (start 165.6 46.35) (end 166.6 47.35) (stroke (width 0.05) (type default)) (layer "Edge.Cuts"))
 (gr_line (start 112.4 100) (end 112.4 35.7) (stroke (width 0.05) (type default)) (layer "Edge.Cuts"))
 (gr_line (start 124.5 112.3) (end 115.6 112.3) (stroke (width 0.05) (type default)) (layer "Edge.Cuts"))
 (gr_line (start 115.35 47.35) (end 116.35 46.35) (stroke (width 0.05) (type default)) (layer "Edge.Cuts"))
 (gr_line (start 115.6 112.3) (end 114.6 111.3) (stroke (width 0.05) (type default)) (layer "Edge.Cuts"))
 (gr_line (start 125.15 95.5) (end 125.95 94.7) (stroke (width 0.05) (type default)) (layer "Edge.Cuts"))
 (gr_line (start 166.6 95.5) (end 166.6 99.45) (stroke (width 0.05) (type default)) (layer "Edge.Cuts"))
 (gr_line (start 125.48 101) (end 113.4 101) (stroke (width 0.05) (type default)) (layer "Edge.Cuts"))
 (gr_line (start 169.5 58.7) (end 171.2 60.4) (stroke (width 0.05) (type default)) (layer "Edge.Cuts"))
 (gr_line (start 168.5 111.8) (end 125 111.8) (stroke (width 0.05) (type default)) (layer "Edge.Cuts"))
 (gr_line (start 171.2 94.9) (end 169.5 96.6) (stroke (width 0.05) (type default)) (layer "Edge.Cuts"))
 (gr_line (start 166.6 99.45) (end 165.8 100.25) (stroke (width 0.05) (type default)) (layer "Edge.Cuts"))
 (gr_line (start 187.8 60.4) (end 189.5 58.7) (stroke (width 0.05) (type default)) (layer "Edge.Cuts"))
 (gr_line (start 202.6 28.5) (end 203.6 29.5) (stroke (width 0.05) (type default)) (layer "Edge.Cuts"))
 (gr_line (start 169.5 35.7) (end 169.5 58.7) (stroke (width 0.05) (type default)) (layer "Edge.Cuts"))
 (gr_line (start 203.6 114.2) (end 202.6 115.2) (stroke (width 0.05) (type default)) (layer "Edge.Cuts"))
 (gr_line (start 114.6 106.5) (end 115.4 105.55) (stroke (width 0.05) (type default)) (layer "Edge.Cuts"))
 (gr_line (start 125.9 104.95) (end 125.9 101.42) (stroke (width 0.05) (type default)) (layer "Edge.Cuts"))
 (gr_line (start 189.5 114.2) (end 189.5 96.6) (stroke (width 0.05) (type default)) (layer "Edge.Cuts"))
 (gr_line (start 203.6 29.5) (end 203.6 114.2) (stroke (width 0.05) (type default)) (layer "Edge.Cuts"))
 (gr_line (start 187.8 94.9) (end 171.2 94.9) (stroke (width 0.05) (type default)) (layer "Edge.Cuts"))
 (gr_line (start 116.35 52) (end 115.35 51) (stroke (width 0.05) (type default)) (layer "Edge.Cuts"))
 (gr_line (start 190.5 28.5) (end 202.6 28.5) (stroke (width 0.05) (type default)) (layer "Edge.Cuts"))
 (segment (start 118.796 40.8) (end 118.796 43.85) (width 0.35) (layer "F.Cu") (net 30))
 (segment (start 121.336 40.8) (end 121.336 43.85) (width 0.35) (layer "F.Cu") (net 31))
 (segment (start 123.876 40.8) (end 123.876 43.85) (width 0.35) (layer "F.Cu") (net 32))
 (segment (start 126.416 40.8) (end 126.416 43.85) (width 0.35) (layer "F.Cu") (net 33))
 (segment (start 128.956 40.8) (end 128.956 43.85) (width 0.35) (layer "F.Cu") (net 34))
 (segment (start 131.496 40.8) (end 131.496 43.85) (width 0.35) (layer "F.Cu") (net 35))
 (segment (start 134.036 40.8) (end 134.036 43.85) (width 0.35) (layer "F.Cu") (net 36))
 (segment (start 136.576 40.8) (end 136.576 43.85) (width 0.35) (layer "F.Cu") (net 37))
 (segment (start 139.116 40.8) (end 139.116 43.85) (width 0.35) (layer "F.Cu") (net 38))
 (segment (start 141.656 40.8) (end 141.656 43.85) (width 0.35) (layer "F.Cu") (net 39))
 (segment (start 145.72 40.8) (end 145.72 43.85) (width 0.35) (layer "F.Cu") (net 5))
 (segment (start 148.26 40.8) (end 148.26 43.85) (width 0.35) (layer "F.Cu") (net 6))
 (segment (start 150.8 40.8) (end 150.8 43.85) (width 0.35) (layer "F.Cu") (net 7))
 (segment (start 153.34 40.8) (end 153.34 43.85) (width 0.35) (layer "F.Cu") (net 8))
 (segment (start 155.88 40.8) (end 155.88 43.85) (width 0.35) (layer "F.Cu") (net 9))
 (segment (start 158.42 40.8) (end 158.42 43.85) (width 0.35) (layer "F.Cu") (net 10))
 (segment (start 160.96 40.8) (end 160.96 43.85) (width 0.35) (layer "F.Cu") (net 11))
 (segment (start 163.5 40.8) (end 163.5 43.85) (width 0.35) (layer "F.Cu") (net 12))
 (segment (start 127.94 106.1) (end 127.94 102.8) (width 0.35) (layer "F.Cu") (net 22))
 (segment (start 130.48 106.1) (end 130.48 102.8) (width 0.5) (layer "F.Cu") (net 23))
 (segment (start 133.02 106.1) (end 133.02 102.8) (width 0.35) (layer "F.Cu") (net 24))
 (segment (start 135.56 106.1) (end 135.56 102.8) (width 0.5) (layer "F.Cu") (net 25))
 (segment (start 138.1 106.1) (end 138.1 102.8) (width 0.5) (layer "F.Cu") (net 26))
 (segment (start 140.64 106.1) (end 140.64 102.8) (width 0.5) (layer "F.Cu") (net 27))
 (segment (start 143.18 106.1) (end 143.18 102.8) (width 0.5) (layer "F.Cu") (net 28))
 (segment (start 145.72 106.1) (end 145.72 102.8) (width 0.5) (layer "F.Cu") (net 29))
 (segment (start 150.8 106.1) (end 150.8 102.8) (width 0.35) (layer "F.Cu") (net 16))
 (segment (start 153.34 106.1) (end 153.34 102.8) (width 0.35) (layer "F.Cu") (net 17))
 (segment (start 155.88 106.1) (end 155.88 102.8) (width 0.35) (layer "F.Cu") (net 18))
 (segment (start 158.42 106.1) (end 158.42 102.8) (width 0.35) (layer "F.Cu") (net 19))
 (segment (start 160.96 106.1) (end 160.96 102.8) (width 0.35) (layer "F.Cu") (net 20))
 (segment (start 163.5 106.1) (end 163.5 102.8) (width 0.35) (layer "F.Cu") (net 21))
 (segment (start 193.5 66.2) (end 196.55 66.2) (width 0.35) (layer "F.Cu") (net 56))
 (segment (start 193.5 68.74) (end 196.55 68.74) (width 0.35) (layer "F.Cu") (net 57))
 (segment (start 193.5 71.28) (end 196.55 71.28) (width 0.35) (layer "F.Cu") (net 58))
 (segment (start 193.5 73.82) (end 196.55 73.82) (width 0.35) (layer "F.Cu") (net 59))
 (segment (start 193.5 76.36) (end 196.55 76.36) (width 0.35) (layer "F.Cu") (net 60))
 (segment (start 193.5 78.9) (end 196.55 78.9) (width 0.35) (layer "F.Cu") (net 61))
 (segment (start 117.78 107.7) (end 117.78 110.7) (width 0.35) (layer "F.Cu") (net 13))
 (segment (start 120.32 107.7) (end 120.32 110.7) (width 0.35) (layer "F.Cu") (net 14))
 (segment (start 122.86 107.7) (end 122.86 110.7) (width 0.35) (layer "F.Cu") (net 15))
 (segment (start 193.5 31.5) (end 196.55 31.5) (width 0.35) (layer "F.Cu") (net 50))
 (segment (start 193.5 34.04) (end 196.55 34.04) (width 0.35) (layer "F.Cu") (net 51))
 (segment (start 193.5 36.58) (end 196.55 36.58) (width 0.35) (layer "F.Cu") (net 52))
 (segment (start 193.5 39.12) (end 196.55 39.12) (width 0.35) (layer "F.Cu") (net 53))
 (segment (start 193.5 41.66) (end 196.55 41.66) (width 0.35) (layer "F.Cu") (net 54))
 (segment (start 193.5 44.2) (end 196.55 44.2) (width 0.35) (layer "F.Cu") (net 55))
 (segment (start 193.5 50.5) (end 196.55 50.5) (width 0.35) (layer "F.Cu") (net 1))
 (segment (start 193.5 53.04) (end 196.55 53.04) (width 0.35) (layer "F.Cu") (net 2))
 (segment (start 193.5 55.58) (end 196.55 55.58) (width 0.35) (layer "F.Cu") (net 3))
 (segment (start 193.5 58.12) (end 196.55 58.12) (width 0.35) (layer "F.Cu") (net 4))
 (segment (start 193.5 89) (end 196.55 89) (width 0.35) (layer "F.Cu") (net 40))
 (segment (start 193.5 91.54) (end 196.55 91.54) (width 0.35) (layer "F.Cu") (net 41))
 (segment (start 193.5 94.08) (end 196.55 94.08) (width 0.35) (layer "F.Cu") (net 42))
 (segment (start 193.5 96.62) (end 196.55 96.62) (width 0.35) (layer "F.Cu") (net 43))
 (segment (start 193.5 99.16) (end 196.55 99.16) (width 0.35) (layer "F.Cu") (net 44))
 (segment (start 193.5 101.7) (end 196.55 101.7) (width 0.35) (layer "F.Cu") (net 45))
 (segment (start 193.5 104.24) (end 196.55 104.24) (width 0.35) (layer "F.Cu") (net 46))
 (segment (start 193.5 106.78) (end 196.55 106.78) (width 0.35) (layer "F.Cu") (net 47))
 (segment (start 193.5 109.32) (end 196.55 109.32) (width 0.35) (layer "F.Cu") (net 48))
 (segment (start 193.5 111.86) (end 196.55 111.86) (width 0.35) (layer "F.Cu") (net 49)))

